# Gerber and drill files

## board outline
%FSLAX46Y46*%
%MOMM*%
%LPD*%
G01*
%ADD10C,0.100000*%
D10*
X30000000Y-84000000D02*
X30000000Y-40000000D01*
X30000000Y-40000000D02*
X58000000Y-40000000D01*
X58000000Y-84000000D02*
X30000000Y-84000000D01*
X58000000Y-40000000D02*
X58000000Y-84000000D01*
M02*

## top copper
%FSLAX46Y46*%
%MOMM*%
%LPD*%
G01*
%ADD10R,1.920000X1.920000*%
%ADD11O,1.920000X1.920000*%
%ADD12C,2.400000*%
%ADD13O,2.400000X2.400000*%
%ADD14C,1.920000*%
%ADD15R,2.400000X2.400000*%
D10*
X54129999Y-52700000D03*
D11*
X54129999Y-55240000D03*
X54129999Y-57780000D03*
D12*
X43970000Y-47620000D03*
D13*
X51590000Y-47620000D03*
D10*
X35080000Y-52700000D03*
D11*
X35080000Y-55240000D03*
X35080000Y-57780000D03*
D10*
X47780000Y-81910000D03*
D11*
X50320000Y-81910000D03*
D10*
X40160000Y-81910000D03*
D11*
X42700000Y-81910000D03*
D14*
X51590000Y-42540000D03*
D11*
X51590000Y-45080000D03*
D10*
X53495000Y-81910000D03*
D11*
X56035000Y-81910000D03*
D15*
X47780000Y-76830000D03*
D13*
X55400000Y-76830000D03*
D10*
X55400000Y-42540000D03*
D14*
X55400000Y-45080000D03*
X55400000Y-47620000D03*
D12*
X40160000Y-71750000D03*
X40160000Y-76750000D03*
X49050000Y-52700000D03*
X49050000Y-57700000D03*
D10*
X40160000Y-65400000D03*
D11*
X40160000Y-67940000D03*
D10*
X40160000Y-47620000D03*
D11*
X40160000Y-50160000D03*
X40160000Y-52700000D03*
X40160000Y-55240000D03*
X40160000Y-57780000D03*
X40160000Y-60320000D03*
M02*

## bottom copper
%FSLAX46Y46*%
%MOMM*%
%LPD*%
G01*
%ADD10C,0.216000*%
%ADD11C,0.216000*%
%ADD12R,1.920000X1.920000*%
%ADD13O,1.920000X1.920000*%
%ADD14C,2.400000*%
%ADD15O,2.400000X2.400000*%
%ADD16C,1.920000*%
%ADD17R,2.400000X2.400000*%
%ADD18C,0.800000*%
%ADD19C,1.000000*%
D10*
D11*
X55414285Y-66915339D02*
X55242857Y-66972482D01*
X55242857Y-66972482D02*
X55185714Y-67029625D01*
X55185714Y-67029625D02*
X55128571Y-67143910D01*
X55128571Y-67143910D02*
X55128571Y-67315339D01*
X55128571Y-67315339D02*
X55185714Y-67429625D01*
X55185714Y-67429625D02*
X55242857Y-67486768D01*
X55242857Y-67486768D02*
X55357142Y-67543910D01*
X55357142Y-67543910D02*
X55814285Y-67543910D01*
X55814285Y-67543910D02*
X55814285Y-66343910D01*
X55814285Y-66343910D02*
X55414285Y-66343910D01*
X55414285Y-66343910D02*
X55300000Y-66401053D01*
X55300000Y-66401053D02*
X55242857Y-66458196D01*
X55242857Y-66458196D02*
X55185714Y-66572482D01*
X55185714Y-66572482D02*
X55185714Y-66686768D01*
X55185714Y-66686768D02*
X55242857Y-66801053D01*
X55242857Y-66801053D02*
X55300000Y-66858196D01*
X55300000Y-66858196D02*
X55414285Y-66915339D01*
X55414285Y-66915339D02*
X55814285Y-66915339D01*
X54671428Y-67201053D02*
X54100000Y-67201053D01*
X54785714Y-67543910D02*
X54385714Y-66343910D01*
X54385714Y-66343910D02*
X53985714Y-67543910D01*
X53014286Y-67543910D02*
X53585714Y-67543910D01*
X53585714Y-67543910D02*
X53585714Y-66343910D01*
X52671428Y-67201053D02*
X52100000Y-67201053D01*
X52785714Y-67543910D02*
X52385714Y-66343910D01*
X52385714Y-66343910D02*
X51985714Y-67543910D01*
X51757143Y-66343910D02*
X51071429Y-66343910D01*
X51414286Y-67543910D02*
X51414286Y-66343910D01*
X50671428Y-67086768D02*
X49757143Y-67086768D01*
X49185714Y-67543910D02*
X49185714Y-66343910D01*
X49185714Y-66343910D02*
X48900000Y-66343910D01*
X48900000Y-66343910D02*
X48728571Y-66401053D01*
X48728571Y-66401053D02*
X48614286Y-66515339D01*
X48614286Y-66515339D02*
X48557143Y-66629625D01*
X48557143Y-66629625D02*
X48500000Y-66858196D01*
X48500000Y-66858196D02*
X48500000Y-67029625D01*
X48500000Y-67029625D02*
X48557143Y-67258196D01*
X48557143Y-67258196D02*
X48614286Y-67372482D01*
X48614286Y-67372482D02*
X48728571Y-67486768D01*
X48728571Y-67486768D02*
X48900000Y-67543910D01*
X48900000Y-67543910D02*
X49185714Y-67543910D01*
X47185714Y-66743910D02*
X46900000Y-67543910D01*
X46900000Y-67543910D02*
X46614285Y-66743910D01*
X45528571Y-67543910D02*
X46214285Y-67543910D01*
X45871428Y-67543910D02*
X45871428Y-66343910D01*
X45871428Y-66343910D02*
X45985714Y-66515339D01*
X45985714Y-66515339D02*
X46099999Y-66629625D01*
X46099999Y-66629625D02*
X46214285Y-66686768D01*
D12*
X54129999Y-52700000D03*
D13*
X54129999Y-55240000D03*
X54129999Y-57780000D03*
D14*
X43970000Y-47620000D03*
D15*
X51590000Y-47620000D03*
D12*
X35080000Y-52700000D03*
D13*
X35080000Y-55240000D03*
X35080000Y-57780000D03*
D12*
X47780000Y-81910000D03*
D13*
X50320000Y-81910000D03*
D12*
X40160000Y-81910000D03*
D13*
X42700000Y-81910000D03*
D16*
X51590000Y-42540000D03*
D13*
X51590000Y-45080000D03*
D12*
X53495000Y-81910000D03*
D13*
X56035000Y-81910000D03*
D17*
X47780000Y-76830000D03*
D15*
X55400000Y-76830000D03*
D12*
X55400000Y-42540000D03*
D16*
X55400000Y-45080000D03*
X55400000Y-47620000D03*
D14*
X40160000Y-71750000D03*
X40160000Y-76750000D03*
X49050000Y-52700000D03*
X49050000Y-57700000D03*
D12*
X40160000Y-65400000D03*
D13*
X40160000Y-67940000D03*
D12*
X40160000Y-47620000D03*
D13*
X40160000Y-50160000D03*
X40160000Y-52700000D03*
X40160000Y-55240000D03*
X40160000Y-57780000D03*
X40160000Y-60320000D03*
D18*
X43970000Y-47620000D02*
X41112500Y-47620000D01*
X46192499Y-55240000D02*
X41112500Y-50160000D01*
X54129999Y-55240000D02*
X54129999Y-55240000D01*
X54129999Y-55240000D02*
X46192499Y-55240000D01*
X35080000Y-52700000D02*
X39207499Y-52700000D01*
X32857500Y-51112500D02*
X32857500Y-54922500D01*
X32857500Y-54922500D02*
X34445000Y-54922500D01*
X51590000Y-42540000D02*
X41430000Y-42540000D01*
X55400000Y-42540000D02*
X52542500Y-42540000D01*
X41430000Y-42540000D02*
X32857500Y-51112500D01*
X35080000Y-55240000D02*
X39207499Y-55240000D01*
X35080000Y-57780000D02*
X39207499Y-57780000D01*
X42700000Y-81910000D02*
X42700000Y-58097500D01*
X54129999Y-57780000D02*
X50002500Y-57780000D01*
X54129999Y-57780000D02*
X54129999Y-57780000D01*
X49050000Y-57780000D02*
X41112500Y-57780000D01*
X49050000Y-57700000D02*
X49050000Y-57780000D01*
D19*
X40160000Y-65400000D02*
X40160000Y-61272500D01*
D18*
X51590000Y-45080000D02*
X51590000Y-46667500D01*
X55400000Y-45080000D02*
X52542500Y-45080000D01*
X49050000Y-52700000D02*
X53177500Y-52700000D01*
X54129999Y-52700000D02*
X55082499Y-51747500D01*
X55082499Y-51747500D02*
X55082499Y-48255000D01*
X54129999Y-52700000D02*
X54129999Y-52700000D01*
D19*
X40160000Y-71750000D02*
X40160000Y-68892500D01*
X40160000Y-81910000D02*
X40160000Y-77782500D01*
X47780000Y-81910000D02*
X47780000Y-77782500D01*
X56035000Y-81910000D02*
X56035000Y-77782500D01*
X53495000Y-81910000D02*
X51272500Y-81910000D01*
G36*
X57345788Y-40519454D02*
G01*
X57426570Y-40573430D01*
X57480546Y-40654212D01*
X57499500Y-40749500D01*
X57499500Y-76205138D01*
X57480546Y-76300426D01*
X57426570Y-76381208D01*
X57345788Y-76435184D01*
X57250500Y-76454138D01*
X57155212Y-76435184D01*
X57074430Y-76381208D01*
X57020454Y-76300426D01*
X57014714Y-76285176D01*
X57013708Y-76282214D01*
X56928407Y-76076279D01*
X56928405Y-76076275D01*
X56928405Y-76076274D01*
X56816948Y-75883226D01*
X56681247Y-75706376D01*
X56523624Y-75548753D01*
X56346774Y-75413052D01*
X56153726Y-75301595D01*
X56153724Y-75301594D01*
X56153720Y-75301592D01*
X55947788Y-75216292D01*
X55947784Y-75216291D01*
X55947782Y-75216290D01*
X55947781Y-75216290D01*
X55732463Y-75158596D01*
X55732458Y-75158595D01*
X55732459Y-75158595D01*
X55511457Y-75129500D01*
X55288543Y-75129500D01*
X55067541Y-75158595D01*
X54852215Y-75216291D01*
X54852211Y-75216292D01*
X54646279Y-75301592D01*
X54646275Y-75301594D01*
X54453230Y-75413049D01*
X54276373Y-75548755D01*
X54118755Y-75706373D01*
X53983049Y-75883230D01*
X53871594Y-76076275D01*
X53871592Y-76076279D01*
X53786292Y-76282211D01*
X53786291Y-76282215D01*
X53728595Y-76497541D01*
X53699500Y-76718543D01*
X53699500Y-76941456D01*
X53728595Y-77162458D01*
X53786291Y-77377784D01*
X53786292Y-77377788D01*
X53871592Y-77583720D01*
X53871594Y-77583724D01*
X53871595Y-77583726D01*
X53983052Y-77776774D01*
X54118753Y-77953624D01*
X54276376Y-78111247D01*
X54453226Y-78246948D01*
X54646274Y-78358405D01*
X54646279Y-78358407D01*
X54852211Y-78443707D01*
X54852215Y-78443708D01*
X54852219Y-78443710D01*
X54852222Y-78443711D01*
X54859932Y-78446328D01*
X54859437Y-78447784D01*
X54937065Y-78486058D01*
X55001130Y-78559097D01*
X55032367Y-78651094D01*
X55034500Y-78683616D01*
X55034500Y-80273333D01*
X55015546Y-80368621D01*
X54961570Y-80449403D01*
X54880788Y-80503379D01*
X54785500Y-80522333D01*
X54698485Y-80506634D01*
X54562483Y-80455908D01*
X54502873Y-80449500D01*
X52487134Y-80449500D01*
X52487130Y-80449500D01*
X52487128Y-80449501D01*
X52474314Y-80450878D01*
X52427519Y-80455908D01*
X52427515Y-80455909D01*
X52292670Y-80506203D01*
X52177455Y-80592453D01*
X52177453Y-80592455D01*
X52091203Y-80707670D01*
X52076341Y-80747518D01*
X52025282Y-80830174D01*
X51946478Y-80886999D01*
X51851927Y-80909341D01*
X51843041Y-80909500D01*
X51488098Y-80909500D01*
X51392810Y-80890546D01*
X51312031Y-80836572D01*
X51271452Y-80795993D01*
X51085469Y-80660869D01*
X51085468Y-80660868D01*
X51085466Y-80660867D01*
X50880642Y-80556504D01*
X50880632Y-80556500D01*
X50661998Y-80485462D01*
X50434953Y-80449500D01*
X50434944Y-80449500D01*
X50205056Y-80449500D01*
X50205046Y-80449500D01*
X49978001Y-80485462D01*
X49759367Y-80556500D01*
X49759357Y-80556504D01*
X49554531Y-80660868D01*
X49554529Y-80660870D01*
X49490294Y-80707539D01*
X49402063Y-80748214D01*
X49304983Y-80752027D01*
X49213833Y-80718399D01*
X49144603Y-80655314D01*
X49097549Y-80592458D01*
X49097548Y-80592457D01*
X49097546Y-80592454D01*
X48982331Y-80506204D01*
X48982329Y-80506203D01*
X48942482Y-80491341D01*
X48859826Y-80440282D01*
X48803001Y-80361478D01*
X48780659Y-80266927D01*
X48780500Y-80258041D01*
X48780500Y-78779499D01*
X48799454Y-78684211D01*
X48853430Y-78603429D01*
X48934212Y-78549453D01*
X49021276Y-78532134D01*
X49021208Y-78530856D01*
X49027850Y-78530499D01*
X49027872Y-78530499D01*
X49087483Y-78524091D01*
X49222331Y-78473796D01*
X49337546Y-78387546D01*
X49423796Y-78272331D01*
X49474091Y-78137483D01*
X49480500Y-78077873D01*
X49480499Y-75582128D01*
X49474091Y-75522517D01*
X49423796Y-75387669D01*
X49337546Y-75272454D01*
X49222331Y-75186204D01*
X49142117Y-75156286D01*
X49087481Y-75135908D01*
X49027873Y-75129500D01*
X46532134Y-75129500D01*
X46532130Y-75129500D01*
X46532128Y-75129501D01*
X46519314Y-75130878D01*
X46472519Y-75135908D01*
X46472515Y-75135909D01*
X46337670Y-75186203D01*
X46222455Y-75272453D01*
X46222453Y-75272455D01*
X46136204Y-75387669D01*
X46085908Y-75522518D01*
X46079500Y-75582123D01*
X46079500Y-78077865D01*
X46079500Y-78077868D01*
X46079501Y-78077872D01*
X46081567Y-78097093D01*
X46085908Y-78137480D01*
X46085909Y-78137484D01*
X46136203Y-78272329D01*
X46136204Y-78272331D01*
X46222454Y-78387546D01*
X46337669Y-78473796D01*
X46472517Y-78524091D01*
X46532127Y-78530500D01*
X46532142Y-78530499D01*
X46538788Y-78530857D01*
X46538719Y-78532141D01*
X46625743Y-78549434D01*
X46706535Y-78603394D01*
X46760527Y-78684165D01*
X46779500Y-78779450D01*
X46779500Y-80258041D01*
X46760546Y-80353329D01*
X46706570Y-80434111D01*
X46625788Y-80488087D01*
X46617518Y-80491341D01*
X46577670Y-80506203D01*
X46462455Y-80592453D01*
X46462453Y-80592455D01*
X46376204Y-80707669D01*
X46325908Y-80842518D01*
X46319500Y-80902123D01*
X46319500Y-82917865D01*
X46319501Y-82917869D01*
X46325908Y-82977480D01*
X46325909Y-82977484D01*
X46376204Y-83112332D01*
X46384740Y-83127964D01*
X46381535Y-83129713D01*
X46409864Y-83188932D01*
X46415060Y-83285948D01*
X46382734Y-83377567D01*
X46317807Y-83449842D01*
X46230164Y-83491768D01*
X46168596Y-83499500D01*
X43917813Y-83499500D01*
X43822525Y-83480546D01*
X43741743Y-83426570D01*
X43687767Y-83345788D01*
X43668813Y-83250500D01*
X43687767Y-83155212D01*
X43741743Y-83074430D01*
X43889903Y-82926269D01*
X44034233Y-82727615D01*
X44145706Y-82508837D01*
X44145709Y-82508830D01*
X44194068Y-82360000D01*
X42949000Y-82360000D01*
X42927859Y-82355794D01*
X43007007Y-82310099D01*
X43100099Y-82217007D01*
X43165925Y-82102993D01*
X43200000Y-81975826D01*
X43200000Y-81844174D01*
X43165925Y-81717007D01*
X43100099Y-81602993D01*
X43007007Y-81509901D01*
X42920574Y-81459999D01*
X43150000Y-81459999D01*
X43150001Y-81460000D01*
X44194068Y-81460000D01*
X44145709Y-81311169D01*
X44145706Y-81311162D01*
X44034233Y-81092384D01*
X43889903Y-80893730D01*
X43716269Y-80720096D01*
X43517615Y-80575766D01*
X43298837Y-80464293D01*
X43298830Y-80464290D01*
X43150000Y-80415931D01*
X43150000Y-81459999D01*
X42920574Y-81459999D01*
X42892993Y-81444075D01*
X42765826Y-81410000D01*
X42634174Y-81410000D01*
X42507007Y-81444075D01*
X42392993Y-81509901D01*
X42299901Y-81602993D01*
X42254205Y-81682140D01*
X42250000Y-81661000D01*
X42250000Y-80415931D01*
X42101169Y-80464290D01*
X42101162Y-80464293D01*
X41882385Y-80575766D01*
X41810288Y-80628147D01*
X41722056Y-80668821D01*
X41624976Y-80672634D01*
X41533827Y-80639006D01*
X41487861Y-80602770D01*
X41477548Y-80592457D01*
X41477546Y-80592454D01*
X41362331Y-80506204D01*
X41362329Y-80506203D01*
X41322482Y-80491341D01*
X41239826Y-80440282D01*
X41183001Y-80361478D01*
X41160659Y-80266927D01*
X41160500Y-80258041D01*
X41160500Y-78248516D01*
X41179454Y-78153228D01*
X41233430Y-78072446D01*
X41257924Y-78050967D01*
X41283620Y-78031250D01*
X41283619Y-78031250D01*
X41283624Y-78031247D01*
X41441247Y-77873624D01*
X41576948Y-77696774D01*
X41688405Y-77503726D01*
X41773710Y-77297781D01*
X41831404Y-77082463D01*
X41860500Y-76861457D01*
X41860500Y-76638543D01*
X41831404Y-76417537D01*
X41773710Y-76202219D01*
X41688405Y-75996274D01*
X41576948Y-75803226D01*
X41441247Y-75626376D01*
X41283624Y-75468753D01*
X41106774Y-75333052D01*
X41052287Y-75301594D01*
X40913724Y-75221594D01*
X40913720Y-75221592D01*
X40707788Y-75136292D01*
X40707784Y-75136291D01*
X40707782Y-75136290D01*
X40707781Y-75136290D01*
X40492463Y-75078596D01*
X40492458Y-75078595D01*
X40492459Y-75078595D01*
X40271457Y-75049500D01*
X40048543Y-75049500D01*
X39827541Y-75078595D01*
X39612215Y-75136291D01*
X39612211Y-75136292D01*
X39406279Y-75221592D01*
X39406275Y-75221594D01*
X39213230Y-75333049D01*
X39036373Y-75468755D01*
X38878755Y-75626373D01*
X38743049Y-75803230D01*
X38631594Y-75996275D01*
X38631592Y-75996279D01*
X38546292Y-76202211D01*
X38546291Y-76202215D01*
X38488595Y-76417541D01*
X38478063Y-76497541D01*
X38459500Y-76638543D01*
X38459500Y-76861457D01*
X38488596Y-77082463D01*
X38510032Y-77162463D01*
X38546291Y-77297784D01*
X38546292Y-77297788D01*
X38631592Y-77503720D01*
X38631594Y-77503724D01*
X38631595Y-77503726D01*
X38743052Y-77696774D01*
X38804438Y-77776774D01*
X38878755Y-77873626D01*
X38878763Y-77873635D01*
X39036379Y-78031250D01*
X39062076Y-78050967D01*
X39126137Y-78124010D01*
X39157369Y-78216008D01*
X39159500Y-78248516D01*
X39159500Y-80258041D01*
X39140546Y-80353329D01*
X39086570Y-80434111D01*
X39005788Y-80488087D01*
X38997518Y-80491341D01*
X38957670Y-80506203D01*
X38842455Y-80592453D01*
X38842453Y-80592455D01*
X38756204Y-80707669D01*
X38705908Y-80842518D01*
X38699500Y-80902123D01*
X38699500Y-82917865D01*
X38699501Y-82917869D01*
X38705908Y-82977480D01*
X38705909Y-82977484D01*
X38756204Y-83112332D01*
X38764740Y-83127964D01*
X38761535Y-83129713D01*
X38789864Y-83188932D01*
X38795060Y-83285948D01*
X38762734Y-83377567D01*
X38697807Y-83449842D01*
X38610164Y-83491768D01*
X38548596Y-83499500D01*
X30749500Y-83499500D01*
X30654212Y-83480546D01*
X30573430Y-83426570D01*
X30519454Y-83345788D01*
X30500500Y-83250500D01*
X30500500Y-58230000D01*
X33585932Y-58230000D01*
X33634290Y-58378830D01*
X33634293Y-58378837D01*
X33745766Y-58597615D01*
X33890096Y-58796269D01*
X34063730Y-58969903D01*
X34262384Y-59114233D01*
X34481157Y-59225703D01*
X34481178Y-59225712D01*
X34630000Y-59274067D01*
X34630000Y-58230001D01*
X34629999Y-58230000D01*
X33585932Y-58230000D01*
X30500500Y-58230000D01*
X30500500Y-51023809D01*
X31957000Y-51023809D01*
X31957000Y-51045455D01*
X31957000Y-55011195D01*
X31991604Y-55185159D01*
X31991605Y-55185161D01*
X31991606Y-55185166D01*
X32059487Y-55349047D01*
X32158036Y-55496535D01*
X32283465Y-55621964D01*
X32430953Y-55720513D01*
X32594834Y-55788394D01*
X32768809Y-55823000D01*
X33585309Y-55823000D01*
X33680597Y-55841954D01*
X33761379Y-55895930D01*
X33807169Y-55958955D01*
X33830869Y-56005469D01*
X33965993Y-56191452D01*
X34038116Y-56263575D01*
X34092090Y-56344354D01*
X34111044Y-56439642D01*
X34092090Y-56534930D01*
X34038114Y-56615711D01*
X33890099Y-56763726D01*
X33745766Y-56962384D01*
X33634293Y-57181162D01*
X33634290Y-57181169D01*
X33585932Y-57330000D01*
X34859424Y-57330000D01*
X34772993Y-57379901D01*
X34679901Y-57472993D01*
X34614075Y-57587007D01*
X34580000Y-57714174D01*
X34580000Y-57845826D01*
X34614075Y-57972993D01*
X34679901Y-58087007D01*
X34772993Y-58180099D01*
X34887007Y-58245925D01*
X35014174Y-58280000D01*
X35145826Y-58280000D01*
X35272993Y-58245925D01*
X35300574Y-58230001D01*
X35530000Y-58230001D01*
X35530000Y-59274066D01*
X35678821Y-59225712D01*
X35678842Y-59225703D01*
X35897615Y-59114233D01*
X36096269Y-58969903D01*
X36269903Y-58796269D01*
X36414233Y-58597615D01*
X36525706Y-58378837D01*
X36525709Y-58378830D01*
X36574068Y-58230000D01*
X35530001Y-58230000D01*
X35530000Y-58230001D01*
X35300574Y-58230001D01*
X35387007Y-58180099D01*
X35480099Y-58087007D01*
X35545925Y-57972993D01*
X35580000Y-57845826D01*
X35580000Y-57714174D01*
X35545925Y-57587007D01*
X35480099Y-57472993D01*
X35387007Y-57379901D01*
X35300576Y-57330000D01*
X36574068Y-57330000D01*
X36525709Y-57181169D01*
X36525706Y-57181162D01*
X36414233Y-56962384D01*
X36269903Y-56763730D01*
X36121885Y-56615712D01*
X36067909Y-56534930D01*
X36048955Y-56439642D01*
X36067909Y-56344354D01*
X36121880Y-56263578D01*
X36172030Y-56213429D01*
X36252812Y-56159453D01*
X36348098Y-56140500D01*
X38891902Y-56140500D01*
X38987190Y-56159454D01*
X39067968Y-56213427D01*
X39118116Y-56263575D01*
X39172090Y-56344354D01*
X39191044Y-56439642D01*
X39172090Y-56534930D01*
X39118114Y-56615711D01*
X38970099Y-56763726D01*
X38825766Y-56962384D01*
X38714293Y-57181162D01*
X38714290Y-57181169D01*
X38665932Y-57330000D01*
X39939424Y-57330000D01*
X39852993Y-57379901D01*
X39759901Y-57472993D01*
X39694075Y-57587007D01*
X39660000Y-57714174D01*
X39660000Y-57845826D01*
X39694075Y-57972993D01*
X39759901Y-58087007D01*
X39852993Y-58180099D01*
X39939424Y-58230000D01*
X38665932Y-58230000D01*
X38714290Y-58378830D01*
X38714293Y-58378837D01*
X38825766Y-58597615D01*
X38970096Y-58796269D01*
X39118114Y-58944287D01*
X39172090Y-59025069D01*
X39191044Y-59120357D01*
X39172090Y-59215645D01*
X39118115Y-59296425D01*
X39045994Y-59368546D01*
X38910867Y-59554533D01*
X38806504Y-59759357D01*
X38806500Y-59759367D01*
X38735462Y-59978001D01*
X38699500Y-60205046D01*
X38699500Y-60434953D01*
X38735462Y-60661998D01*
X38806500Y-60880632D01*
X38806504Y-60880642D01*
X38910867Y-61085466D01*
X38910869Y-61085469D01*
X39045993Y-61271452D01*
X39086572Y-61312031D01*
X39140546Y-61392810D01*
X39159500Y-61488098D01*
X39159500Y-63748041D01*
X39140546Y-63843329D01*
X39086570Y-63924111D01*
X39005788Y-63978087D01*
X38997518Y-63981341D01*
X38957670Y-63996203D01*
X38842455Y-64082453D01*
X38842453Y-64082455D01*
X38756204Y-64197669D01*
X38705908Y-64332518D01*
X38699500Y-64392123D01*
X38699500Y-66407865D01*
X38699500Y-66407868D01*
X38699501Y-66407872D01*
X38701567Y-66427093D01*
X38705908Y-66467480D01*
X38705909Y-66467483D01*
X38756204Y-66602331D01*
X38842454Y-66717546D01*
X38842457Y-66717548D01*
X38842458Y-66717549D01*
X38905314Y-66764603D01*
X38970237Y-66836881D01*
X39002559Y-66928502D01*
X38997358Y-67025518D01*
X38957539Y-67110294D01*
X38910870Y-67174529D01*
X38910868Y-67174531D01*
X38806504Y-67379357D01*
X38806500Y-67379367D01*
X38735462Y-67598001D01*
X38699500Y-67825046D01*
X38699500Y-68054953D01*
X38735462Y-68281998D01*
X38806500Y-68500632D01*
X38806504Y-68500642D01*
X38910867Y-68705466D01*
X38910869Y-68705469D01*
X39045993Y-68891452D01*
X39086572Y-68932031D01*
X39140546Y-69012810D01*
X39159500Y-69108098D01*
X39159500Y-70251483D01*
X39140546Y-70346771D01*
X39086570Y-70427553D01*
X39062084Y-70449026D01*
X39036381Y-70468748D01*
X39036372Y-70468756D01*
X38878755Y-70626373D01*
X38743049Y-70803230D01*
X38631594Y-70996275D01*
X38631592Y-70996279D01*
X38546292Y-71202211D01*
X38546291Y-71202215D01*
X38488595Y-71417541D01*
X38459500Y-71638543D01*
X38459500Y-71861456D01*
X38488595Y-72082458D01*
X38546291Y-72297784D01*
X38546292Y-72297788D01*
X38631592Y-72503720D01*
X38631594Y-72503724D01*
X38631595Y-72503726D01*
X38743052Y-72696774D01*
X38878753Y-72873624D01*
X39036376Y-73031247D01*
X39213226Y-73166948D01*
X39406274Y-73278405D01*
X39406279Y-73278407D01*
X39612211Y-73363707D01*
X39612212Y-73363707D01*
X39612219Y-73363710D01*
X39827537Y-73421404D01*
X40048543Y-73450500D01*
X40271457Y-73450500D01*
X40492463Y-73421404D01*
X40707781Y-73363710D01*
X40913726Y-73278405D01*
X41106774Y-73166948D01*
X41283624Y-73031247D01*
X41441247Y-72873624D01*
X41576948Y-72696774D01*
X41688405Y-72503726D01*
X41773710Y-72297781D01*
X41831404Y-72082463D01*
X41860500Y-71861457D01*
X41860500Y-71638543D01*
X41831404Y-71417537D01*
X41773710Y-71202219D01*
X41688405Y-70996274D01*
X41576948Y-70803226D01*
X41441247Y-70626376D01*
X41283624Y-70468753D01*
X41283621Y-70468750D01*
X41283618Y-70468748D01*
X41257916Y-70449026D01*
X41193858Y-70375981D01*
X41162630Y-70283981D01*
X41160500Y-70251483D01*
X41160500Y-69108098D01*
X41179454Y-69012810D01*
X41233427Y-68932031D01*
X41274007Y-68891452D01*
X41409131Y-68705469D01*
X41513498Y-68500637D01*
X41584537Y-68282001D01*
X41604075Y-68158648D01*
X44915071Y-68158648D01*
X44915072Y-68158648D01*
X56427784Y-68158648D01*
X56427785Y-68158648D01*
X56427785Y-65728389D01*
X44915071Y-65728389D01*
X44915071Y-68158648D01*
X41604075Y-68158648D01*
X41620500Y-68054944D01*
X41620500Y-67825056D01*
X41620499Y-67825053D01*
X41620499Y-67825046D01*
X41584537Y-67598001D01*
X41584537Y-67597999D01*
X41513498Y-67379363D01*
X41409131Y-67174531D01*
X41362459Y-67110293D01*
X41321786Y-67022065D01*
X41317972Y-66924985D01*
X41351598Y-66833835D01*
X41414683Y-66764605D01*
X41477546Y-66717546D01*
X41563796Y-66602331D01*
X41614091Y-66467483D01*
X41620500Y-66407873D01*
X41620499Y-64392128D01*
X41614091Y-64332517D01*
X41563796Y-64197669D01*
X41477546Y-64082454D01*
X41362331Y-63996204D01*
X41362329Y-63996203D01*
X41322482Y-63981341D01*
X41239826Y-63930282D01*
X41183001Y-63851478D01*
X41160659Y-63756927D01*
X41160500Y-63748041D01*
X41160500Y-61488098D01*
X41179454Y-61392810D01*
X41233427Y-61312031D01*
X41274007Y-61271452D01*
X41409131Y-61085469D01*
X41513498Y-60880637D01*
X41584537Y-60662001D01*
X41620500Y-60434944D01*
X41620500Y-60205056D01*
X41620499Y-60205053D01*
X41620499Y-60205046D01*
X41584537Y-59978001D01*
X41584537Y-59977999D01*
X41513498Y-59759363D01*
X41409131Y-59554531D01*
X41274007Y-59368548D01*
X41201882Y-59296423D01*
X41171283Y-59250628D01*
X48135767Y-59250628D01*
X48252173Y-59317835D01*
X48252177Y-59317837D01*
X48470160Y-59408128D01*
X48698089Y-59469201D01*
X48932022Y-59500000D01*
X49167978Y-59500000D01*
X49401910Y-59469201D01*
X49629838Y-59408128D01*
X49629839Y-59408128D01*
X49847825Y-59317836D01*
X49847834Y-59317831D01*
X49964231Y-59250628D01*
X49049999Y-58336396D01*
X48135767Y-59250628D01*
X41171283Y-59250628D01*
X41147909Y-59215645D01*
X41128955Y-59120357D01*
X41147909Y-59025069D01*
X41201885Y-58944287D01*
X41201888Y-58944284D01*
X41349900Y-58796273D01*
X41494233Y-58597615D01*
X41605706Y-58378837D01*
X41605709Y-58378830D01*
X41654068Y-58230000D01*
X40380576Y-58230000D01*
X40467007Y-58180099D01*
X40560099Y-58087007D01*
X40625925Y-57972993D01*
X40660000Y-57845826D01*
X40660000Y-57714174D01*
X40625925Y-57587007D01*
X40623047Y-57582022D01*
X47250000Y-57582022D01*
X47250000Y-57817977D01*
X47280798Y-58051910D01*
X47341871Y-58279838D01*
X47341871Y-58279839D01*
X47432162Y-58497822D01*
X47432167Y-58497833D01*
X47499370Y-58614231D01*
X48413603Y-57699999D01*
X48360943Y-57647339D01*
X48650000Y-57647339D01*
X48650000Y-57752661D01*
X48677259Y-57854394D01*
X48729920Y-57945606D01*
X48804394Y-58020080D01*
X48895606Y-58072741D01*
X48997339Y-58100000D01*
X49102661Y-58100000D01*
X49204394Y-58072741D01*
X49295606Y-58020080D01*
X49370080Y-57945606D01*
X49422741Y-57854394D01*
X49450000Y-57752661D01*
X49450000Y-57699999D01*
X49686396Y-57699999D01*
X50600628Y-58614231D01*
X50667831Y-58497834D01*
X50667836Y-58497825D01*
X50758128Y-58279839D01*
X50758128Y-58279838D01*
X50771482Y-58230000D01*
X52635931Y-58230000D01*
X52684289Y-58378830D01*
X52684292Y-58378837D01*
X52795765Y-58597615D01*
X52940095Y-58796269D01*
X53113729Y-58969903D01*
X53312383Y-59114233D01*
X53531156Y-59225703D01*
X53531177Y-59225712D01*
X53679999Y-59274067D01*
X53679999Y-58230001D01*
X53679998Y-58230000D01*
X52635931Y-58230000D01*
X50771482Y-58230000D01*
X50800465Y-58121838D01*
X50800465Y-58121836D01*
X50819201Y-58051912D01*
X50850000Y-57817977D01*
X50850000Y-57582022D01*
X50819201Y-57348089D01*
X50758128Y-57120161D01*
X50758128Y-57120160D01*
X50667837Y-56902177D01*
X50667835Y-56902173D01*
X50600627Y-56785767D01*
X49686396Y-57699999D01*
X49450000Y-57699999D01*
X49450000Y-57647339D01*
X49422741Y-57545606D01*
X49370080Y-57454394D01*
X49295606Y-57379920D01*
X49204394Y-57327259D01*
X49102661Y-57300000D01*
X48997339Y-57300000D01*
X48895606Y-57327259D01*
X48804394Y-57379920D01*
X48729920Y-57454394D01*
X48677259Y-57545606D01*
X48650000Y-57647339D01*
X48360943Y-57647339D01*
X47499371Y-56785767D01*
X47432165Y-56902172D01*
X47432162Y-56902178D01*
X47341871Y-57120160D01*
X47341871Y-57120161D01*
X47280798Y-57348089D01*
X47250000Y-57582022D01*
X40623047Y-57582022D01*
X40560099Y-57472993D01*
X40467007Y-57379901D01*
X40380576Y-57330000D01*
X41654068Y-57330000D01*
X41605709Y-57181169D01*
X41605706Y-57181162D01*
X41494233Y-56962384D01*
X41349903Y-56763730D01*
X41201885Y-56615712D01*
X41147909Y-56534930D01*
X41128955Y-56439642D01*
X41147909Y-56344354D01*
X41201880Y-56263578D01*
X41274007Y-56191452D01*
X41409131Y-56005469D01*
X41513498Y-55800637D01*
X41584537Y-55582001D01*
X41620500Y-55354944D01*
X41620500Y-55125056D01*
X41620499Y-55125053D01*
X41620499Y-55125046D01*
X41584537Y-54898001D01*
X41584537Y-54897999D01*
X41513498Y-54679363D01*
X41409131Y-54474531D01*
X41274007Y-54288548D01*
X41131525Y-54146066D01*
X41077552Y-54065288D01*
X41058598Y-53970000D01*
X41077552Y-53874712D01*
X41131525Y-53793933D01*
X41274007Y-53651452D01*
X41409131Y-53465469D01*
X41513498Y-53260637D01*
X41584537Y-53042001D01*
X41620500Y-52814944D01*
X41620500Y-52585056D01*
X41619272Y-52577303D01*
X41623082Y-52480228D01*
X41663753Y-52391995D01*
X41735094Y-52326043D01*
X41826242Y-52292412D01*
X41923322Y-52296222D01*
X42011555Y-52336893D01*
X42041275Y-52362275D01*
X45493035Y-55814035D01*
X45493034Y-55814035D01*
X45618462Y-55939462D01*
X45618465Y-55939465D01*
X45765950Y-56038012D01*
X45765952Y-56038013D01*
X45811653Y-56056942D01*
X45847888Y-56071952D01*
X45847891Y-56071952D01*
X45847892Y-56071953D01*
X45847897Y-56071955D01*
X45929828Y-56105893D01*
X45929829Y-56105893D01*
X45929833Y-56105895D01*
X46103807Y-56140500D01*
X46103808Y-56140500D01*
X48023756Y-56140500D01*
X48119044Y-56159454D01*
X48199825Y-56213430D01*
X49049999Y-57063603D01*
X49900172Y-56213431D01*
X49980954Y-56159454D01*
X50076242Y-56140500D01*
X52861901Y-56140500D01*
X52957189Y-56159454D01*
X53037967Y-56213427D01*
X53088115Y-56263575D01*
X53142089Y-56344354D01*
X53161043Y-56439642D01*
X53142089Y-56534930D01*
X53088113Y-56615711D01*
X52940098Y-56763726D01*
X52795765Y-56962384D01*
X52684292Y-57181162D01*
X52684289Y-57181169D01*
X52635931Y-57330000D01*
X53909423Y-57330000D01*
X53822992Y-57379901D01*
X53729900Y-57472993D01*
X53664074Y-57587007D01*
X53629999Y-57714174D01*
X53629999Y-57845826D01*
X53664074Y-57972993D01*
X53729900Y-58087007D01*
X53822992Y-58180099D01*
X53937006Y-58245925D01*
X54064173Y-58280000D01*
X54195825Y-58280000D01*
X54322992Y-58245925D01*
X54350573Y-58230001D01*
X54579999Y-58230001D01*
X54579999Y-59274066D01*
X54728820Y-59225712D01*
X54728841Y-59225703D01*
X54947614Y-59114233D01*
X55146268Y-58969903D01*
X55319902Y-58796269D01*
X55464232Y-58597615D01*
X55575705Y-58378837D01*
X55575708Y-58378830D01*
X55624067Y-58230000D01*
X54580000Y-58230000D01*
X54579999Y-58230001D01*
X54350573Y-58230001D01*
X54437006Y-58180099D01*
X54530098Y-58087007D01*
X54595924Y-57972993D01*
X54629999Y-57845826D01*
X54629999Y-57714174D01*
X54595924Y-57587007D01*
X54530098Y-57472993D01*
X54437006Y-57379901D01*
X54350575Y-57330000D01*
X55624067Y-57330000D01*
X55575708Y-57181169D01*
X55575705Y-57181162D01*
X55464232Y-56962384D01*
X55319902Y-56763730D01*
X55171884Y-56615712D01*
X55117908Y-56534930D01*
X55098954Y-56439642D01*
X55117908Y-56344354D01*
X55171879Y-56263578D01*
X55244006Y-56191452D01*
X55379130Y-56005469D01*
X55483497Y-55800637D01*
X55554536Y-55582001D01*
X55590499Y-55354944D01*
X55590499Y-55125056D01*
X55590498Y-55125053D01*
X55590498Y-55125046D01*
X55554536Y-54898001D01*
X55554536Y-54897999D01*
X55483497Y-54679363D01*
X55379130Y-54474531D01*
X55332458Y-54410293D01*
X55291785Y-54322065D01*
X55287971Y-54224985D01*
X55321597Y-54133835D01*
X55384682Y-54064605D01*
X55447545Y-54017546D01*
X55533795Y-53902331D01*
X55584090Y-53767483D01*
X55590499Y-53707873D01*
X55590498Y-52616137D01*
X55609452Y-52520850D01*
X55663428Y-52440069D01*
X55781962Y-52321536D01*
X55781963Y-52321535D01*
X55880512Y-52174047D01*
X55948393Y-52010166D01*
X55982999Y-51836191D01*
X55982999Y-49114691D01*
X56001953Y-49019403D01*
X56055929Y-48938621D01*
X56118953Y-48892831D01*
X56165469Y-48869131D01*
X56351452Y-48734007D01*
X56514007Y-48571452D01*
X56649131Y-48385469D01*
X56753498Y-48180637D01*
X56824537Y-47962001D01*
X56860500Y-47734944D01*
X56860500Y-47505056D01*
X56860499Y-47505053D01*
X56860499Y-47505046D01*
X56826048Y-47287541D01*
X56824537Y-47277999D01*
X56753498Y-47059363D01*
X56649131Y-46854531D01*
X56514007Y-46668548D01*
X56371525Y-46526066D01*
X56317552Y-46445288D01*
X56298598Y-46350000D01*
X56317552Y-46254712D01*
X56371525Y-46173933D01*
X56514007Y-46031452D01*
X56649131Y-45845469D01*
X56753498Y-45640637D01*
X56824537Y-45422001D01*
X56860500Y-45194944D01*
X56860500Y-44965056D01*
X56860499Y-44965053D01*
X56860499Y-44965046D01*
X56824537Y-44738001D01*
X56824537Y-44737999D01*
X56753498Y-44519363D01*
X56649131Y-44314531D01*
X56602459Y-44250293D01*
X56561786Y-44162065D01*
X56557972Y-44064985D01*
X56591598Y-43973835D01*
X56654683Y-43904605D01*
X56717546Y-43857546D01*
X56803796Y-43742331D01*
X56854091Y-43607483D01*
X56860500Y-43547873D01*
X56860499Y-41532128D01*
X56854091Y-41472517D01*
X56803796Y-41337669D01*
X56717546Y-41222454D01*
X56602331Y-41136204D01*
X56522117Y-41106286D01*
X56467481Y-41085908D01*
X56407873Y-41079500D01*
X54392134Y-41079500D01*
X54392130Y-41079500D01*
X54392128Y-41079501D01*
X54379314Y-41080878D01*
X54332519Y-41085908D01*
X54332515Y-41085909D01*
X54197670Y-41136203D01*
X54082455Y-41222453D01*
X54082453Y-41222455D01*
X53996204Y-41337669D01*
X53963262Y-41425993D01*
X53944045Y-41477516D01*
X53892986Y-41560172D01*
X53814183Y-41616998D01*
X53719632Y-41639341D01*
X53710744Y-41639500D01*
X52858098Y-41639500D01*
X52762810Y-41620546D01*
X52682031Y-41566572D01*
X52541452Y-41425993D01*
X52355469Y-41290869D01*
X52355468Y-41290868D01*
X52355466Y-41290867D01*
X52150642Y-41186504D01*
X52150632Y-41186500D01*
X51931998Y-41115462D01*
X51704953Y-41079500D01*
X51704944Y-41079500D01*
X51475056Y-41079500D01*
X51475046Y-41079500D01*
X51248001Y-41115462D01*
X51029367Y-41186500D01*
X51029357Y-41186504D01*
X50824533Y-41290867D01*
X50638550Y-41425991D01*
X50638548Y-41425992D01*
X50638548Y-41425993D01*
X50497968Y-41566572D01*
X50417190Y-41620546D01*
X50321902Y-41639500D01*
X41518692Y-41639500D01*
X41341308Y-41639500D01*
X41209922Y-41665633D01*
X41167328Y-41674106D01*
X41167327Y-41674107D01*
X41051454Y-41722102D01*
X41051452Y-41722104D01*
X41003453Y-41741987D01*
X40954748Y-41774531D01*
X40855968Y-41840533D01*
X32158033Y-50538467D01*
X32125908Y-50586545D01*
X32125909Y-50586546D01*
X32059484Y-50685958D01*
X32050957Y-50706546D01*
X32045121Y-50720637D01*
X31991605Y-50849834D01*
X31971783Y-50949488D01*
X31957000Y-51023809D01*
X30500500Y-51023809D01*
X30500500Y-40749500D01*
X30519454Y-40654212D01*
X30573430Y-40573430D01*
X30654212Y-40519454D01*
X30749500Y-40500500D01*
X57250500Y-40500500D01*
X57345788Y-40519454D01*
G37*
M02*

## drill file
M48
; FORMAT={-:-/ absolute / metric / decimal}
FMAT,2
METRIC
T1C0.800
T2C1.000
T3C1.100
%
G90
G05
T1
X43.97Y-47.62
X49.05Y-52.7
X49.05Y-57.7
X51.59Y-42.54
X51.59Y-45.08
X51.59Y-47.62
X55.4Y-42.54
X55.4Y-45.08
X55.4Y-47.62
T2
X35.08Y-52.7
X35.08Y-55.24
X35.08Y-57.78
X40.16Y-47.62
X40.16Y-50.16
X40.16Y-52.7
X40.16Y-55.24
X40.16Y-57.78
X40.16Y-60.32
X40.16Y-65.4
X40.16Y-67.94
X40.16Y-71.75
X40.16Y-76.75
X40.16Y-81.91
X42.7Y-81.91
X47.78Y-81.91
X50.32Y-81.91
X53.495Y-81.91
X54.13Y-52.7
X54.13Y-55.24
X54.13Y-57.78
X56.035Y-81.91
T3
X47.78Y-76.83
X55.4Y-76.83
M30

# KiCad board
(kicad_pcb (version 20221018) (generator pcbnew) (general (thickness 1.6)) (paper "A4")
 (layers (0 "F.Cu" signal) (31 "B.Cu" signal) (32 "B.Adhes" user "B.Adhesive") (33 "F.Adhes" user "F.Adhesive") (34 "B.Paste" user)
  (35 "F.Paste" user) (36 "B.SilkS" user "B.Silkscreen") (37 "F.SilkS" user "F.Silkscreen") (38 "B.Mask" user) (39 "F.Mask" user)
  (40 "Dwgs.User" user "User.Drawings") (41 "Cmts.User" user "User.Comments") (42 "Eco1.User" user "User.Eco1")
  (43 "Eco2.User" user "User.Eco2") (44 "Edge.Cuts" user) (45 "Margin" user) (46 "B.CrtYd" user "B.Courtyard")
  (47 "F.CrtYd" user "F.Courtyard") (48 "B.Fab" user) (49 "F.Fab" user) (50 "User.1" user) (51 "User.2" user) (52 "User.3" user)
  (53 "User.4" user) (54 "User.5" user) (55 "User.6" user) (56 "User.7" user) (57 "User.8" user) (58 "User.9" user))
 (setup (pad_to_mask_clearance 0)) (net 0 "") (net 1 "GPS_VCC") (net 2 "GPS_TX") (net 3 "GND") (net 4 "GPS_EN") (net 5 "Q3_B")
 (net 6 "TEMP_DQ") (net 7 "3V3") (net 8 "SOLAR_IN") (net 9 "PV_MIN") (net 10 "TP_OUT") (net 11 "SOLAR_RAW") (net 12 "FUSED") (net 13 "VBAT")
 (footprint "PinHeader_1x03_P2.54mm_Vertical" (layer "F.Cu") (at 54.129999 52.7)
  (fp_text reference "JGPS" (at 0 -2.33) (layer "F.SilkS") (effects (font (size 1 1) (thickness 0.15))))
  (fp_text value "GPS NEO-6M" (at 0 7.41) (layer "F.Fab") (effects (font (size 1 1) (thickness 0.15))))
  (pad "1" thru_hole rect (at 0 0) (size 1.92 1.92) (drill 1) (layers "*.Cu" "*.Mask") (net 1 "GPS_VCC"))
  (pad "2" thru_hole oval (at 0 2.54) (size 1.92 1.92) (drill 1) (layers "*.Cu" "*.Mask") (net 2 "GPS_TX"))
  (pad "3" thru_hole oval (at 0 5.08) (size 1.92 1.92) (drill 1) (layers "*.Cu" "*.Mask") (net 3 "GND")))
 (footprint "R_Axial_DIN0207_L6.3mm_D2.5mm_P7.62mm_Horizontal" (layer "F.Cu") (at 43.97 47.62)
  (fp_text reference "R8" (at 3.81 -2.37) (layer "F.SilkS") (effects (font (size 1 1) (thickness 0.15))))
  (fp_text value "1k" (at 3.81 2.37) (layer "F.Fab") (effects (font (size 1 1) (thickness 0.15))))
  (pad "1" thru_hole circle (at 0 0) (size 2.4 2.4) (drill 0.8) (layers "*.Cu" "*.Mask") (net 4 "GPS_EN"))
  (pad "2" thru_hole oval (at 7.62 0) (size 2.4 2.4) (drill 0.8) (layers "*.Cu" "*.Mask") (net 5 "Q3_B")))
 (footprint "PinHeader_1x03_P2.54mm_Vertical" (layer "F.Cu") (at 35.08 52.7)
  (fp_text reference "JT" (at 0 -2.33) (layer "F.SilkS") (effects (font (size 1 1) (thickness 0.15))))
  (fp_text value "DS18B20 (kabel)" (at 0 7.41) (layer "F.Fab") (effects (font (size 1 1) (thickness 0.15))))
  (pad "1" thru_hole rect (at 0 0) (size 1.92 1.92) (drill 1) (layers "*.Cu" "*.Mask") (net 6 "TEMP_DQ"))
  (pad "2" thru_hole oval (at 0 2.54) (size 1.92 1.92) (drill 1) (layers "*.Cu" "*.Mask") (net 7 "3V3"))
  (pad "3" thru_hole oval (at 0 5.08) (size 1.92 1.92) (drill 1) (layers "*.Cu" "*.Mask") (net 3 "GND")))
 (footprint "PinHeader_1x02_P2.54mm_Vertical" (layer "F.Cu") (at 47.78 81.91 90)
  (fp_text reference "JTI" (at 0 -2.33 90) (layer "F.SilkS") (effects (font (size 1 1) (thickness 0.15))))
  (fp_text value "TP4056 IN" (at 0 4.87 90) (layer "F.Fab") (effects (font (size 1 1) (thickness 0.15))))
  (pad "1" thru_hole rect (at 0 0 90) (size 1.92 1.92) (drill 1) (layers "*.Cu" "*.Mask") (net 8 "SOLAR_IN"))
  (pad "2" thru_hole oval (at 0 2.54 90) (size 1.92 1.92) (drill 1) (layers "*.Cu" "*.Mask") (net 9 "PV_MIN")))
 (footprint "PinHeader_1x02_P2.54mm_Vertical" (layer "F.Cu") (at 40.16 81.91 90)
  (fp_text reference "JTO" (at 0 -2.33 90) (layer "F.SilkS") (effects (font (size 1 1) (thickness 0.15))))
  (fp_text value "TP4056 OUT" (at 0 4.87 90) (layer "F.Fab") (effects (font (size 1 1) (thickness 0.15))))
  (pad "1" thru_hole rect (at 0 0 90) (size 1.92 1.92) (drill 1) (layers "*.Cu" "*.Mask") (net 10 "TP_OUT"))
  (pad "2" thru_hole oval (at 0 2.54 90) (size 1.92 1.92) (drill 1) (layers "*.Cu" "*.Mask") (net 3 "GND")))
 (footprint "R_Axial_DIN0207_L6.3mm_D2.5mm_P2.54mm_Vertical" (layer "F.Cu") (at 51.59 42.54 -90)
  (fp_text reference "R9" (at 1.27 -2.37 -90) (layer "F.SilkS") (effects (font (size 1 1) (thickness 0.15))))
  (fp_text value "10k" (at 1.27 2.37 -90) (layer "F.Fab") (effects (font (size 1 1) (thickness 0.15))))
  (pad "1" thru_hole circle (at 0 0 270) (size 1.92 1.92) (drill 0.8) (layers "*.Cu" "*.Mask") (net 7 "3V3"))
  (pad "2" thru_hole oval (at 2.54 0 270) (size 1.92 1.92) (drill 0.8) (layers "*.Cu" "*.Mask") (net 5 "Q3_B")))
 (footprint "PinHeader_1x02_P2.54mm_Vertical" (layer "F.Cu") (at 53.495 81.91 90)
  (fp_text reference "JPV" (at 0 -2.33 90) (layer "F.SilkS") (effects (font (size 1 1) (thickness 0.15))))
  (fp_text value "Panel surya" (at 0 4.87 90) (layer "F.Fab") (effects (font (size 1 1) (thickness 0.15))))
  (pad "1" thru_hole rect (at 0 0 90) (size 1.92 1.92) (drill 1) (layers "*.Cu" "*.Mask") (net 9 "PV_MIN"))
  (pad "2" thru_hole oval (at 0 2.54 90) (size 1.92 1.92) (drill 1) (layers "*.Cu" "*.Mask") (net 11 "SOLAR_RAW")))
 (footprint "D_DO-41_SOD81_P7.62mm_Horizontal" (layer "F.Cu") (at 47.78 76.83)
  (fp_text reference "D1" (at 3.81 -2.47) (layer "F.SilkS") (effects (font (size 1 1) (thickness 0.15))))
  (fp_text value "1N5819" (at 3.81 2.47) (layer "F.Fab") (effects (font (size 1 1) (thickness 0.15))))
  (pad "1" thru_hole rect (at 0 0) (size 2.4 2.4) (drill 1.1) (layers "*.Cu" "*.Mask") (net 8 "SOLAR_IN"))
  (pad "2" thru_hole oval (at 7.62 0) (size 2.4 2.4) (drill 1.1) (layers "*.Cu" "*.Mask") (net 11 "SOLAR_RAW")))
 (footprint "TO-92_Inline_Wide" (layer "F.Cu") (at 55.4 42.54 -90)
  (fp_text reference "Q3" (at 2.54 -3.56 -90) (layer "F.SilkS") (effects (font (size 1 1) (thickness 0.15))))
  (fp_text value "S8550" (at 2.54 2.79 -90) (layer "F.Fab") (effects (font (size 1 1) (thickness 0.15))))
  (pad "1" thru_hole rect (at 0 0 270) (size 1.92 1.92) (drill 0.8) (layers "*.Cu" "*.Mask") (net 7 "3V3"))
  (pad "2" thru_hole circle (at 2.54 0 270) (size 1.92 1.92) (drill 0.8) (layers "*.Cu" "*.Mask") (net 5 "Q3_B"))
  (pad "3" thru_hole circle (at 5.08 0 270) (size 1.92 1.92) (drill 0.8) (layers "*.Cu" "*.Mask") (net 1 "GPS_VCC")))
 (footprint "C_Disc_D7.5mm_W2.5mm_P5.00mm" (layer "F.Cu") (at 40.16 71.75 -90)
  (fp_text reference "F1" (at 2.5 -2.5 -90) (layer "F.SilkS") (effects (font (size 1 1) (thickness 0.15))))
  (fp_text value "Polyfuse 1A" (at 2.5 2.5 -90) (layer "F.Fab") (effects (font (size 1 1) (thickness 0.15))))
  (pad "1" thru_hole circle (at 0 0 270) (size 2.4 2.4) (drill 1) (layers "*.Cu" "*.Mask") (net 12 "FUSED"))
  (pad "2" thru_hole circle (at 5 0 270) (size 2.4 2.4) (drill 1) (layers "*.Cu" "*.Mask") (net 10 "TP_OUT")))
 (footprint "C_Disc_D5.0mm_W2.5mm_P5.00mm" (layer "F.Cu") (at 49.05 52.7 -90)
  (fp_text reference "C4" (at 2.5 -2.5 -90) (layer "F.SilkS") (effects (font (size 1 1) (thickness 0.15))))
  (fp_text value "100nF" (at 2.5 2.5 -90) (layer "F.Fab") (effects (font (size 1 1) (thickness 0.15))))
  (pad "1" thru_hole circle (at 0 0 270) (size 2.4 2.4) (drill 0.8) (layers "*.Cu" "*.Mask") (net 1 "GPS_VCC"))
  (pad "2" thru_hole circle (at 5 0 270) (size 2.4 2.4) (drill 0.8) (layers "*.Cu" "*.Mask") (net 3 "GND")))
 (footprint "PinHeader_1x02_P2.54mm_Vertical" (layer "F.Cu") (at 40.16 65.4)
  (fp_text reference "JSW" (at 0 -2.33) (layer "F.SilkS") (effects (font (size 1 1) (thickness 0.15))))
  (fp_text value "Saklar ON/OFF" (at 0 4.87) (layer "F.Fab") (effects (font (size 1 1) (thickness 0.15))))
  (pad "1" thru_hole rect (at 0 0) (size 1.92 1.92) (drill 1) (layers "*.Cu" "*.Mask") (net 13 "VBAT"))
  (pad "2" thru_hole oval (at 0 2.54) (size 1.92 1.92) (drill 1) (layers "*.Cu" "*.Mask") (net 12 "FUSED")))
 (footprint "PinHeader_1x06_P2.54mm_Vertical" (layer "F.Cu") (at 40.16 47.62)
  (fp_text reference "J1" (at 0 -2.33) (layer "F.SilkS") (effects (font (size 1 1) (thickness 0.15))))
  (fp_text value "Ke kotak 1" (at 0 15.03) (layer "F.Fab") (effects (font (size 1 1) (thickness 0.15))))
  (pad "1" thru_hole rect (at 0 0) (size 1.92 1.92) (drill 1) (layers "*.Cu" "*.Mask") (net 4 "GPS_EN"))
  (pad "2" thru_hole oval (at 0 2.54) (size 1.92 1.92) (drill 1) (layers "*.Cu" "*.Mask") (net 2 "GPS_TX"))
  (pad "3" thru_hole oval (at 0 5.08) (size 1.92 1.92) (drill 1) (layers "*.Cu" "*.Mask") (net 6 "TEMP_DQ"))
  (pad "4" thru_hole oval (at 0 7.62) (size 1.92 1.92) (drill 1) (layers "*.Cu" "*.Mask") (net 7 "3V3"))
  (pad "5" thru_hole oval (at 0 10.16) (size 1.92 1.92) (drill 1) (layers "*.Cu" "*.Mask") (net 3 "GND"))
  (pad "6" thru_hole oval (at 0 12.7) (size 1.92 1.92) (drill 1) (layers "*.Cu" "*.Mask") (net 13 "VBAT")))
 (gr_line (start 30 84) (end 30 40) (stroke (width 0.1) (type default)) (layer "Edge.Cuts"))
 (gr_line (start 30 40) (end 58 40) (stroke (width 0.1) (type default)) (layer "Edge.Cuts"))
 (gr_line (start 58 84) (end 30 84) (stroke (width 0.1) (type default)) (layer "Edge.Cuts"))
 (gr_line (start 58 40) (end 58 84) (stroke (width 0.1) (type default)) (layer "Edge.Cuts"))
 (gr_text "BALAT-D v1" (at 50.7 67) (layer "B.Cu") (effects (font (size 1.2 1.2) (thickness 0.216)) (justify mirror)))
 (segment (start 43.97 47.62) (end 41.1125 47.62) (width 0.8) (layer "B.Cu") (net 4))
 (segment (start 46.192499 55.24) (end 41.1125 50.16) (width 0.8) (layer "B.Cu") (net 2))
 (segment (start 54.129999 55.24) (end 54.129999 55.24) (width 0.8) (layer "B.Cu") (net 2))
 (segment (start 54.129999 55.24) (end 46.192499 55.24) (width 0.8) (layer "B.Cu") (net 2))
 (segment (start 35.08 52.7) (end 39.207499 52.7) (width 0.8) (layer "B.Cu") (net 6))
 (segment (start 32.8575 51.1125) (end 32.8575 54.9225) (width 0.8) (layer "B.Cu") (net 7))
 (segment (start 32.8575 54.9225) (end 34.445 54.9225) (width 0.8) (layer "B.Cu") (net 7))
 (segment (start 51.59 42.54) (end 41.43 42.54) (width 0.8) (layer "B.Cu") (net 7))
 (segment (start 55.4 42.54) (end 52.5425 42.54) (width 0.8) (layer "B.Cu") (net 7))
 (segment (start 41.43 42.54) (end 32.8575 51.1125) (width 0.8) (layer "B.Cu") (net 7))
 (segment (start 35.08 55.24) (end 39.207499 55.24) (width 0.8) (layer "B.Cu") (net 7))
 (segment (start 35.08 57.78) (end 39.207499 57.78) (width 0.8) (layer "B.Cu") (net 3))
 (segment (start 42.7 81.91) (end 42.7 58.0975) (width 0.8) (layer "B.Cu") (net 3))
 (segment (start 54.129999 57.78) (end 50.0025 57.78) (width 0.8) (layer "B.Cu") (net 3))
 (segment (start 54.129999 57.78) (end 54.129999 57.78) (width 0.8) (layer "B.Cu") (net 3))
 (segment (start 49.05 57.78) (end 41.1125 57.78) (width 0.8) (layer "B.Cu") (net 3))
 (segment (start 49.05 57.7) (end 49.05 57.78) (width 0.8) (layer "B.Cu") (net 3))
 (segment (start 40.16 65.4) (end 40.16 61.2725) (width 1) (layer "B.Cu") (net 13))
 (segment (start 51.59 45.08) (end 51.59 46.6675) (width 0.8) (layer "B.Cu") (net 5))
 (segment (start 55.4 45.08) (end 52.5425 45.08) (width 0.8) (layer "B.Cu") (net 5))
 (segment (start 49.05 52.7) (end 53.1775 52.7) (width 0.8) (layer "B.Cu") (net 1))
 (segment (start 54.129999 52.7) (end 55.082499 51.7475) (width 0.8) (layer "B.Cu") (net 1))
 (segment (start 55.082499 51.7475) (end 55.082499 48.255) (width 0.8) (layer "B.Cu") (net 1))
 (segment (start 54.129999 52.7) (end 54.129999 52.7) (width 0.8) (layer "B.Cu") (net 1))
 (segment (start 40.16 71.75) (end 40.16 68.8925) (width 1) (layer "B.Cu") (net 12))
 (segment (start 40.16 81.91) (end 40.16 77.7825) (width 1) (layer "B.Cu") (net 10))
 (segment (start 47.78 81.91) (end 47.78 77.7825) (width 1) (layer "B.Cu") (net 8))
 (segment (start 56.035 81.91) (end 56.035 77.7825) (width 1) (layer "B.Cu") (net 11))
 (segment (start 53.495 81.91) (end 51.2725 81.91) (width 1) (layer "B.Cu") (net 9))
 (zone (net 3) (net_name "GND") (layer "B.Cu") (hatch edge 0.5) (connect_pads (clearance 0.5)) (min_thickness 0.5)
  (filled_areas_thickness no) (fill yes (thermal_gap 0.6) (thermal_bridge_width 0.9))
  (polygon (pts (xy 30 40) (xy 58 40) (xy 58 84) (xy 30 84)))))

